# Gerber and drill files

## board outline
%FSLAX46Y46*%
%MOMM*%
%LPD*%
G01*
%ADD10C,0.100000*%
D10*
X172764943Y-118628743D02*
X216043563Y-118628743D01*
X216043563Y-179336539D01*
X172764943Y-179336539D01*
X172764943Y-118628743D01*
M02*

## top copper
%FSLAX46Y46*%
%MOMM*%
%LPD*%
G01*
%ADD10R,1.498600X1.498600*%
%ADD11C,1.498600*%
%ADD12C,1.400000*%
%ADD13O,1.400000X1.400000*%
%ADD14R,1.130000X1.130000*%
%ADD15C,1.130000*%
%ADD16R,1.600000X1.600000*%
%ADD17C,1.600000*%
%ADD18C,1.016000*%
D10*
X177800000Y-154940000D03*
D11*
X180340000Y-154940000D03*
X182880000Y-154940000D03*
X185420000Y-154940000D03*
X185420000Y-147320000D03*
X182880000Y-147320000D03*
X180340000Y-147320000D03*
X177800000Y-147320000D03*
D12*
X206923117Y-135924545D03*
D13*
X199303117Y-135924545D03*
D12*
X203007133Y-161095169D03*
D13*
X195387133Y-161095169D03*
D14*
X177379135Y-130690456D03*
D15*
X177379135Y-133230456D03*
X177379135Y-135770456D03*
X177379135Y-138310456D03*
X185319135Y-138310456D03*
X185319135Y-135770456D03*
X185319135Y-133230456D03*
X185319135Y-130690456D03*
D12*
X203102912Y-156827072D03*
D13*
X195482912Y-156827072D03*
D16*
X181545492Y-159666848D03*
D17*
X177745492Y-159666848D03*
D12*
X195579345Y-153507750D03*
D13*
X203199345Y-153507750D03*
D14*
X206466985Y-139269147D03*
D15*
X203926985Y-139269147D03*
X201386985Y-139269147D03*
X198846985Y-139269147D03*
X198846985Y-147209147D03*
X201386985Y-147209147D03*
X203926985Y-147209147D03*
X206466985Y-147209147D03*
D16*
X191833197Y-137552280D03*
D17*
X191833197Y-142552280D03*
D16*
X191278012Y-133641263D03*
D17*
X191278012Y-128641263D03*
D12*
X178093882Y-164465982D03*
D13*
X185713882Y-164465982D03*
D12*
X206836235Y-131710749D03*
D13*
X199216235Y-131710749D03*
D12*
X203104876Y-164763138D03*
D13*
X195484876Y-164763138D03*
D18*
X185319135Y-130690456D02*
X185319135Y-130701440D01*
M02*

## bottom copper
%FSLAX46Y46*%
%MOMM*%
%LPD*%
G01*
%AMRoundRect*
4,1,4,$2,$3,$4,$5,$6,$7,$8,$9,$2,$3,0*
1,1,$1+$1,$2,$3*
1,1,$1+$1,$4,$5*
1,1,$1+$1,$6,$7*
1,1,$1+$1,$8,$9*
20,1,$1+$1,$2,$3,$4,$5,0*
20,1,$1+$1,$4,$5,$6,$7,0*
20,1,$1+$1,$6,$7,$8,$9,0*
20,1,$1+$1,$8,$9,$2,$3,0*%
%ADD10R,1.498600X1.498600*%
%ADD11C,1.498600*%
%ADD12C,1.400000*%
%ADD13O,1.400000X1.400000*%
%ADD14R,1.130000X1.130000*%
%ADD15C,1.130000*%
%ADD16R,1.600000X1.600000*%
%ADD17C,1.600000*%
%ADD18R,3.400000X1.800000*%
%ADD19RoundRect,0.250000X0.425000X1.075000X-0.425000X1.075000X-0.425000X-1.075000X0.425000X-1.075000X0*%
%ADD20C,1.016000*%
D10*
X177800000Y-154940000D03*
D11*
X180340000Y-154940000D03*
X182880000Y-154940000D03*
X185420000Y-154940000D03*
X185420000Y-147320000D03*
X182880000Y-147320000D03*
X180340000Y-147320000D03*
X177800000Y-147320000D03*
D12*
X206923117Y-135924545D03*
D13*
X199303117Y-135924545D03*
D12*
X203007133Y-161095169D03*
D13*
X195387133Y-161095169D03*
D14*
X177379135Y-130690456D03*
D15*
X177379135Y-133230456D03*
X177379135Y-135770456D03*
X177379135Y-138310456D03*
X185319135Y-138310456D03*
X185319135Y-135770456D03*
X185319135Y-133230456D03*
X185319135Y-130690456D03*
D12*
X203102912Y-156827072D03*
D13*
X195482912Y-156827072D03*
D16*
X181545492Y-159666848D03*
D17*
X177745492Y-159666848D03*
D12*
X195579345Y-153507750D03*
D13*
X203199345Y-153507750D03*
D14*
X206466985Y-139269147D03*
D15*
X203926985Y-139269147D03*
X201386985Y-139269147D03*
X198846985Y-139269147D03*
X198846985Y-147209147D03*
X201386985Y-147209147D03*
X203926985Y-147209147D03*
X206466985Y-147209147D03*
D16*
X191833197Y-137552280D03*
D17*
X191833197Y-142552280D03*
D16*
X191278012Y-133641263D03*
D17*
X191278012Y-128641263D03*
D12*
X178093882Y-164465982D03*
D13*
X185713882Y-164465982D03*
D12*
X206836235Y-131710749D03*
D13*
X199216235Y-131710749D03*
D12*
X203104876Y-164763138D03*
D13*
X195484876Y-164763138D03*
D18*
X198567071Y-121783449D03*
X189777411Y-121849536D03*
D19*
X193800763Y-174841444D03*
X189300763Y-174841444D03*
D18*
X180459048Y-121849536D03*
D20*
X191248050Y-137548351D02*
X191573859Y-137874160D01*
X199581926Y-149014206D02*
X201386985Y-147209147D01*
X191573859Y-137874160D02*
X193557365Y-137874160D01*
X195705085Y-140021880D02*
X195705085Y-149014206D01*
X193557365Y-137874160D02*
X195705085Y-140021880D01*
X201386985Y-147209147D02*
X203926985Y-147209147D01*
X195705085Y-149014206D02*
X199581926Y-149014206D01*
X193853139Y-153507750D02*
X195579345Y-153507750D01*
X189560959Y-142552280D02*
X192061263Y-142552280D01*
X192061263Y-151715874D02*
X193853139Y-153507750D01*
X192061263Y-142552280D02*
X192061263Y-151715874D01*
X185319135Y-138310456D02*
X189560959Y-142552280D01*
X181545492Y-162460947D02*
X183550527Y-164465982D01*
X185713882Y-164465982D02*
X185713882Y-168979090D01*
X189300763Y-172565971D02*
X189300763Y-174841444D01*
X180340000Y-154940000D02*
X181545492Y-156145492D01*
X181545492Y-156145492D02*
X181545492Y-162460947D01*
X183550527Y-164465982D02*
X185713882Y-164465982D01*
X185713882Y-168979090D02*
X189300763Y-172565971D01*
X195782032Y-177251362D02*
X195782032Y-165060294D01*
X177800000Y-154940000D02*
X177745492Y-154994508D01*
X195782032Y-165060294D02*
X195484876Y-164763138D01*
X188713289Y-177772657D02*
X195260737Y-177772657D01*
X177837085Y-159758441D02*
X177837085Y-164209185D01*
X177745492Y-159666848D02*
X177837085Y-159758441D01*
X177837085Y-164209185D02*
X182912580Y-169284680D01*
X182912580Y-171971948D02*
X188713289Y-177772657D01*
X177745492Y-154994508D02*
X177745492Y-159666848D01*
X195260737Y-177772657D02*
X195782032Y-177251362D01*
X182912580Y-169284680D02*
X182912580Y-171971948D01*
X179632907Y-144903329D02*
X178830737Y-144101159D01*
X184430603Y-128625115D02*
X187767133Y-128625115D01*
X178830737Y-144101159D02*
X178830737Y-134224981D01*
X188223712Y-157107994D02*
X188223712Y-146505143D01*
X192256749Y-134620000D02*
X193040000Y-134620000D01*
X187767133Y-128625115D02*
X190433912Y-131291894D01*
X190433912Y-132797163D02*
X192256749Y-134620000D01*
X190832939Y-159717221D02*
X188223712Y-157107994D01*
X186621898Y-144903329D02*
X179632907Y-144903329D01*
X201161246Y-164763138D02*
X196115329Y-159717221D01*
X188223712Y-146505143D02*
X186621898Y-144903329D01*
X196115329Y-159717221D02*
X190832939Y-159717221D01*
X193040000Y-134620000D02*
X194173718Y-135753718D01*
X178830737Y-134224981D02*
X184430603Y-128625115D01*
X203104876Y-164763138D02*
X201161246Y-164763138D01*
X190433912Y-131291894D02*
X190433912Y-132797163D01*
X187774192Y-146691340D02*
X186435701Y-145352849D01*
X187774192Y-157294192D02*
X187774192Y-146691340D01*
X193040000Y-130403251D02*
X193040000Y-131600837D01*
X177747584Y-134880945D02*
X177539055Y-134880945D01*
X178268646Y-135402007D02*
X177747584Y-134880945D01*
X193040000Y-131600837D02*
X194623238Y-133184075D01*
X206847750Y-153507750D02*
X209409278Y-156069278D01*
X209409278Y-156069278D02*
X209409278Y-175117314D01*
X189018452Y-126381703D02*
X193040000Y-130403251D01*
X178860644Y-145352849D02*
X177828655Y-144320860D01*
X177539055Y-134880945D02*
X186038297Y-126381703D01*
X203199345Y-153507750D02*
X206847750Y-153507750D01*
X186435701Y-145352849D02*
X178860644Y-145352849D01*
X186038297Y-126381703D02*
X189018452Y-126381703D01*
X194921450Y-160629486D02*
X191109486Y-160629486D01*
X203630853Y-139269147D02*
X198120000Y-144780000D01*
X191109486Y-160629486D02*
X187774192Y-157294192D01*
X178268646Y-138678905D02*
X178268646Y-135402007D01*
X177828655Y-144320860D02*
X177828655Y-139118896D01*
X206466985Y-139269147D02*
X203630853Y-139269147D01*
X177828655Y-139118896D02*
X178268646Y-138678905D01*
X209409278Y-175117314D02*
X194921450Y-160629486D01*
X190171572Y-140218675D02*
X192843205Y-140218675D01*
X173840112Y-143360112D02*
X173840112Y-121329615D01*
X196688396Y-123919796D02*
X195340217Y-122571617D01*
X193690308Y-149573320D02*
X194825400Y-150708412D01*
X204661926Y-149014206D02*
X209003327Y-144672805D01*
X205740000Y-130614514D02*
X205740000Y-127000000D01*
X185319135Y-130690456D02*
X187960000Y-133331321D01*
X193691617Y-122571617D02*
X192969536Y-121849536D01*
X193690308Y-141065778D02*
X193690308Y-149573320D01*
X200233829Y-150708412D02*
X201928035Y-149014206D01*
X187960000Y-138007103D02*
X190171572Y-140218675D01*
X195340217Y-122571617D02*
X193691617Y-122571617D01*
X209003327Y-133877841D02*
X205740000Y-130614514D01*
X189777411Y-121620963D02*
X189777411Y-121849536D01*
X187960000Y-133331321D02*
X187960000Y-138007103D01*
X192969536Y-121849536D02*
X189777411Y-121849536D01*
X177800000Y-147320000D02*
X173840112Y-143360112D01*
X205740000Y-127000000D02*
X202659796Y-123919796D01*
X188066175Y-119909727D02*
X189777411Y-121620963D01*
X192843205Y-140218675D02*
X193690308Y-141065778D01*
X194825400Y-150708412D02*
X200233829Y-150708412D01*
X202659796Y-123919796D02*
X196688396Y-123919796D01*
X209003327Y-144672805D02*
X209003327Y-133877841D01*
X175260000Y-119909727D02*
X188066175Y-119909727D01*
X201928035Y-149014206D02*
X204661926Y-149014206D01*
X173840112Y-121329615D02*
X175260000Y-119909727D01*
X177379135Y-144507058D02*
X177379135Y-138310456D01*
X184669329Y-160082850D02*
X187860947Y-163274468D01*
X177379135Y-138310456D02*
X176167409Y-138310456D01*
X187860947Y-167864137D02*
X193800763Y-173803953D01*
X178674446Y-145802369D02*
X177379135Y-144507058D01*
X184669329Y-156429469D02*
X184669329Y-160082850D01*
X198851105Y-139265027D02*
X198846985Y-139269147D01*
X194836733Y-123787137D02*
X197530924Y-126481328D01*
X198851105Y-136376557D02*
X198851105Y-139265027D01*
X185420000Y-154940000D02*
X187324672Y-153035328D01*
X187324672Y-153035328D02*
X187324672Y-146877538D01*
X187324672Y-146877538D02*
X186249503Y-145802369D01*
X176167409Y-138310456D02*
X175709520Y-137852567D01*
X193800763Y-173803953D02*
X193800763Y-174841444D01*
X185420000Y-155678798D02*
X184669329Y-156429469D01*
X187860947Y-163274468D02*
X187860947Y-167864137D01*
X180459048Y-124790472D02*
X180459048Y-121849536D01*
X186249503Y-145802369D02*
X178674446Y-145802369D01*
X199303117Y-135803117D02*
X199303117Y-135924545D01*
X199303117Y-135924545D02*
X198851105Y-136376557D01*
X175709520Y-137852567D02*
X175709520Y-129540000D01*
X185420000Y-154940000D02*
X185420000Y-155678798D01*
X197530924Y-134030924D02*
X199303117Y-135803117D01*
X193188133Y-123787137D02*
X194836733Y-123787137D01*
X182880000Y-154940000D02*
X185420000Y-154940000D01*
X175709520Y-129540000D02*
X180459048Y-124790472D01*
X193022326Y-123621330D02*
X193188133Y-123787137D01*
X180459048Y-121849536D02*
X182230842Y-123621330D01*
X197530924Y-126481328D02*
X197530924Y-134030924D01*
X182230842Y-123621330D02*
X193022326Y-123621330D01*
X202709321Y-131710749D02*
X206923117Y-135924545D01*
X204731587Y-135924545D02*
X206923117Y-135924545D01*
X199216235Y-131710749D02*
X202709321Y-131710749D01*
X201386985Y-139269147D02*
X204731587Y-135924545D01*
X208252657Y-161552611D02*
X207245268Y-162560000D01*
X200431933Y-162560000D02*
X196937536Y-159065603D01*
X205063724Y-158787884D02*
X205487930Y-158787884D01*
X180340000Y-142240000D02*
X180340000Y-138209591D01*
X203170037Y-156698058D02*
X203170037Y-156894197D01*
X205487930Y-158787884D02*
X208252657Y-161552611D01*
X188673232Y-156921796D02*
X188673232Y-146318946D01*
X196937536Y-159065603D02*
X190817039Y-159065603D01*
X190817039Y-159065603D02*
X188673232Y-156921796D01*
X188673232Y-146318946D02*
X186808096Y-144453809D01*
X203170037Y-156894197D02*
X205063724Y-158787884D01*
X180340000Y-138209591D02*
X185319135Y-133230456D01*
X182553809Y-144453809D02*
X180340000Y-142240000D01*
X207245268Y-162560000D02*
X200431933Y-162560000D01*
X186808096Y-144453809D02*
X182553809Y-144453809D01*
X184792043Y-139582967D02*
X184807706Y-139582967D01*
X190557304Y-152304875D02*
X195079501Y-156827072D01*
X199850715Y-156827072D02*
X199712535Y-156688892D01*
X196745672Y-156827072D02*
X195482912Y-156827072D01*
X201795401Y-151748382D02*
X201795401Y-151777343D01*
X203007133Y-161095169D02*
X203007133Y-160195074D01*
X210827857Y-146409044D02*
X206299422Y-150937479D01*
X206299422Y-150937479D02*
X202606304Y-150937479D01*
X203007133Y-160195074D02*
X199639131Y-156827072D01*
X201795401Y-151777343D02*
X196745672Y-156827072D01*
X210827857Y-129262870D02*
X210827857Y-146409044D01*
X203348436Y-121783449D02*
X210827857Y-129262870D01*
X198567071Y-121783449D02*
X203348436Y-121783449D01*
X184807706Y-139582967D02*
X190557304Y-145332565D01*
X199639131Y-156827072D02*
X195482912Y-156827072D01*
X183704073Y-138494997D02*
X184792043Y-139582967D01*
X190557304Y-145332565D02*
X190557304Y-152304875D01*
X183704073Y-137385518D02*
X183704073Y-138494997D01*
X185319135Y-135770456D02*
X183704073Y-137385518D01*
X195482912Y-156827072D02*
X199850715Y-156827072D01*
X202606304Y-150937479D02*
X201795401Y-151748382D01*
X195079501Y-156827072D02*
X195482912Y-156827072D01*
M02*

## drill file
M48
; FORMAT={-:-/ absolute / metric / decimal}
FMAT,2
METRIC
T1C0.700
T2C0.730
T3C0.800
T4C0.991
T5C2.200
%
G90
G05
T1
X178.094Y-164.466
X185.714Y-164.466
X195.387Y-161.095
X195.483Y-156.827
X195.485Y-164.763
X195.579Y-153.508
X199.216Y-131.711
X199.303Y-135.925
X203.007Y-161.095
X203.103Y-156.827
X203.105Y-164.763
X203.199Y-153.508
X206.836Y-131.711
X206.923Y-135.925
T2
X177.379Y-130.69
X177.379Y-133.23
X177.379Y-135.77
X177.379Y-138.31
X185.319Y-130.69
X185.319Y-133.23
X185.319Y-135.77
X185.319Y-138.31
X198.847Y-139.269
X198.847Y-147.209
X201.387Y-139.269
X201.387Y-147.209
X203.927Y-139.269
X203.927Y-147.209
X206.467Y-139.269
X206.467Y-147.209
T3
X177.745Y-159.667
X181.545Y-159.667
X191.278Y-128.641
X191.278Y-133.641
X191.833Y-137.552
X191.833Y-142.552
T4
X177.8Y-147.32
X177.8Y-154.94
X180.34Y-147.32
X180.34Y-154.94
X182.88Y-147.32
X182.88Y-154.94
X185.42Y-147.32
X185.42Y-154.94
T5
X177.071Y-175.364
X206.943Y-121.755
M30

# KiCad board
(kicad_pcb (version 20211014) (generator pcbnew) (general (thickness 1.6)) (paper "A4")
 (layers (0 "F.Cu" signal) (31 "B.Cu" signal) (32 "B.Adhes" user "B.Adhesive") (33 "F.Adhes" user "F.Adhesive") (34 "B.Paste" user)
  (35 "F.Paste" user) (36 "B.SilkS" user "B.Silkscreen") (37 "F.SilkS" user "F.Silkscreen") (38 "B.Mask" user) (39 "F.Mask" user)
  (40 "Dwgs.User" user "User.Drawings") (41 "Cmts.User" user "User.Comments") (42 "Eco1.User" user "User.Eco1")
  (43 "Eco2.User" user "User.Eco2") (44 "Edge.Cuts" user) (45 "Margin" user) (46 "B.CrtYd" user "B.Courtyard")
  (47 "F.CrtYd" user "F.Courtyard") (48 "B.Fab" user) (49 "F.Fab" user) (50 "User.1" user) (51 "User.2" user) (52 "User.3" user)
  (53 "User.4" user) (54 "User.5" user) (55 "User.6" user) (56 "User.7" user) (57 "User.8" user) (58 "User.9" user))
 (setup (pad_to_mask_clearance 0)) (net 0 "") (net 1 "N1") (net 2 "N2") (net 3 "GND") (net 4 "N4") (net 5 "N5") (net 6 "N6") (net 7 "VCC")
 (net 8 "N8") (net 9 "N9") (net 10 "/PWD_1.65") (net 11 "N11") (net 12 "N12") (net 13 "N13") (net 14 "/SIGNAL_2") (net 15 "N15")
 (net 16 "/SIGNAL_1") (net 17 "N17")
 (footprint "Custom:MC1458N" (layer "F.Cu") (at 177.8 154.94 90)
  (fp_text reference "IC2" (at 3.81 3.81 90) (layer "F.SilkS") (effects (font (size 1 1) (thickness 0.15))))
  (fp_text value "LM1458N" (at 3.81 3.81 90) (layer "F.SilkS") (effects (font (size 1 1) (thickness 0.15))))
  (pad "1" thru_hole rect locked (at 0 0 90) (size 1.4986 1.4986) (drill 0.9906) (layers *.Cu *.Mask) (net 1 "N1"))
  (pad "2" thru_hole circle locked (at 0 2.54 90) (size 1.4986 1.4986) (drill 0.9906) (layers *.Cu *.Mask) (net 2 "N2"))
  (pad "3" thru_hole circle locked (at 0 5.08 90) (size 1.4986 1.4986) (drill 0.9906) (layers *.Cu *.Mask) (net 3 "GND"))
  (pad "4" thru_hole circle locked (at 0 7.62 90) (size 1.4986 1.4986) (drill 0.9906) (layers *.Cu *.Mask) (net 3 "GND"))
  (pad "5" thru_hole circle locked (at 7.62 7.62 90) (size 1.4986 1.4986) (drill 0.9906) (layers *.Cu *.Mask) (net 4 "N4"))
  (pad "6" thru_hole circle locked (at 7.62 5.08 90) (size 1.4986 1.4986) (drill 0.9906) (layers *.Cu *.Mask) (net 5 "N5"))
  (pad "7" thru_hole circle locked (at 7.62 2.54 90) (size 1.4986 1.4986) (drill 0.9906) (layers *.Cu *.Mask) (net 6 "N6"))
  (pad "8" thru_hole circle locked (at 7.62 0 90) (size 1.4986 1.4986) (drill 0.9906) (layers *.Cu *.Mask) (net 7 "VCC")))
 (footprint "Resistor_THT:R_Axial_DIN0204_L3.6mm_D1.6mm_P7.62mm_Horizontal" (layer "F.Cu") (at 206.923117 135.924545 180)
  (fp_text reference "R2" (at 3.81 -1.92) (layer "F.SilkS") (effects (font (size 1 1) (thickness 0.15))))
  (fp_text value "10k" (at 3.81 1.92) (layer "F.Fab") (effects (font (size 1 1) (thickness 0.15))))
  (pad "1" thru_hole circle (at 0 0 180) (size 1.4 1.4) (drill 0.7) (layers *.Cu *.Mask) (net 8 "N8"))
  (pad "2" thru_hole oval (at 7.62 0 180) (size 1.4 1.4) (drill 0.7) (layers *.Cu *.Mask) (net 3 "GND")))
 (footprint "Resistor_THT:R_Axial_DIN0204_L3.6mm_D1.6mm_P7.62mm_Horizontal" (layer "F.Cu") (at 203.007133 161.095169 180)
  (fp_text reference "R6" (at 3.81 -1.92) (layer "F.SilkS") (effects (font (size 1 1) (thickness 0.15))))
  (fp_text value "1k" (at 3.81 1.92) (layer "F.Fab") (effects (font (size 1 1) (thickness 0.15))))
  (pad "1" thru_hole circle (at 0 0 180) (size 1.4 1.4) (drill 0.7) (layers *.Cu *.Mask) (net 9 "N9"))
  (pad "2" thru_hole oval (at 7.62 0 180) (size 1.4 1.4) (drill 0.7) (layers *.Cu *.Mask) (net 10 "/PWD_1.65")))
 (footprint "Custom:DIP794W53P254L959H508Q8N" (layer "F.Cu") (at 181.349135 134.500456)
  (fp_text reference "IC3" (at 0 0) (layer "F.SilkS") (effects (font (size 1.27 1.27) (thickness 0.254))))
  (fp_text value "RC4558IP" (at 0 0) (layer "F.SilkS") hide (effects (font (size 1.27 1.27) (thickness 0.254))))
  (pad "1" thru_hole rect locked (at -3.97 -3.81) (size 1.13 1.13) (drill 0.73) (layers *.Cu *.Mask) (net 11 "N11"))
  (pad "2" thru_hole circle locked (at -3.97 -1.27) (size 1.13 1.13) (drill 0.73) (layers *.Cu *.Mask) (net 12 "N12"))
  (pad "3" thru_hole circle locked (at -3.97 1.27) (size 1.13 1.13) (drill 0.73) (layers *.Cu *.Mask) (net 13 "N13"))
  (pad "4" thru_hole circle locked (at -3.97 3.81) (size 1.13 1.13) (drill 0.73) (layers *.Cu *.Mask) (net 3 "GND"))
  (pad "5" thru_hole circle locked (at 3.97 3.81) (size 1.13 1.13) (drill 0.73) (layers *.Cu *.Mask) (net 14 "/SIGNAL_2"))
  (pad "6" thru_hole circle locked (at 3.97 1.27) (size 1.13 1.13) (drill 0.73) (layers *.Cu *.Mask) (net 9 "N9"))
  (pad "7" thru_hole circle locked (at 3.97 -1.27) (size 1.13 1.13) (drill 0.73) (layers *.Cu *.Mask) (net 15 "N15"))
  (pad "8" thru_hole circle locked (at 3.97 -3.81) (size 1.13 1.13) (drill 0.73) (layers *.Cu *.Mask) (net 7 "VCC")))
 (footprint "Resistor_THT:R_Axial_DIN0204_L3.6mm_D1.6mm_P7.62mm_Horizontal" (layer "F.Cu") (at 203.102912 156.827072 180)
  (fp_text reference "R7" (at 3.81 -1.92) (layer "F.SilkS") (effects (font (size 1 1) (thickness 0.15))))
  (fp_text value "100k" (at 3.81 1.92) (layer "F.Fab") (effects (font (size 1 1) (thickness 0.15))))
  (pad "1" thru_hole circle (at 0 0 180) (size 1.4 1.4) (drill 0.7) (layers *.Cu *.Mask) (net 15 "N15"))
  (pad "2" thru_hole oval (at 7.62 0 180) (size 1.4 1.4) (drill 0.7) (layers *.Cu *.Mask) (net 9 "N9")))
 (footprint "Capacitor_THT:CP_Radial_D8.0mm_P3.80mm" (layer "F.Cu") (at 181.545492 159.666848 180)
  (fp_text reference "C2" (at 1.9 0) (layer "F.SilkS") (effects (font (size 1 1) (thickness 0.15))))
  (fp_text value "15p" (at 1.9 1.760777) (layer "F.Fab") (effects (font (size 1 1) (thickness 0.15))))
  (pad "1" thru_hole rect (at 0 0 180) (size 1.6 1.6) (drill 0.8) (layers *.Cu *.Mask) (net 2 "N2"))
  (pad "2" thru_hole circle (at 3.8 0 180) (size 1.6 1.6) (drill 0.8) (layers *.Cu *.Mask) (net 1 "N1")))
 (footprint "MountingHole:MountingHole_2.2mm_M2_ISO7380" (layer "F.Cu") (at 206.942704 121.75478)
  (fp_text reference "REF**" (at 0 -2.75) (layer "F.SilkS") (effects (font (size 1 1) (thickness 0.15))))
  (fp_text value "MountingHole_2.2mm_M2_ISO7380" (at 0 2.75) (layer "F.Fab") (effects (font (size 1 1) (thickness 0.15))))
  (pad "" np_thru_hole circle (at 0 0) (size 2.2 2.2) (drill 2.2) (layers *.Cu *.Mask)))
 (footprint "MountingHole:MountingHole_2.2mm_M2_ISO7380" (layer "F.Cu") (at 177.071075 175.363506)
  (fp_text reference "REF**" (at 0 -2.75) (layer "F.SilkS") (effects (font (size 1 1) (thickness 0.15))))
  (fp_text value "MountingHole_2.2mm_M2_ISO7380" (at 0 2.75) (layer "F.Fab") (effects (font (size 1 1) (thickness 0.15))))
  (pad "" np_thru_hole circle (at 0 0) (size 2.2 2.2) (drill 2.2) (layers *.Cu *.Mask)))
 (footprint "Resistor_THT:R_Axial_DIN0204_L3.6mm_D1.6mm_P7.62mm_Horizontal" (layer "F.Cu") (at 195.579345 153.50775)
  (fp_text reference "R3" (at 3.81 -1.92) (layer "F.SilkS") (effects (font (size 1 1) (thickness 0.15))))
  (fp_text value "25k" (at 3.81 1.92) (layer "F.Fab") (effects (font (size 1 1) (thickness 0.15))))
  (pad "1" thru_hole circle (at 0 0) (size 1.4 1.4) (drill 0.7) (layers *.Cu *.Mask) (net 14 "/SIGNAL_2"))
  (pad "2" thru_hole oval (at 7.62 0) (size 1.4 1.4) (drill 0.7) (layers *.Cu *.Mask) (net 10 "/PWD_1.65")))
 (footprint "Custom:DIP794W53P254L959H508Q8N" (layer "F.Cu") (at 202.656985 143.239147 -90)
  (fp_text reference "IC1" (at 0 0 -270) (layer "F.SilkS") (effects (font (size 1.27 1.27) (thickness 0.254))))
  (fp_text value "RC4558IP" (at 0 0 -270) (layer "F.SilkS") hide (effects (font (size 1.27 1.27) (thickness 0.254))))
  (pad "1" thru_hole rect locked (at -3.97 -3.81 270) (size 1.13 1.13) (drill 0.73) (layers *.Cu *.Mask) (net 10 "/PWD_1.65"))
  (pad "2" thru_hole circle locked (at -3.97 -1.27 270) (size 1.13 1.13) (drill 0.73) (layers *.Cu *.Mask) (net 10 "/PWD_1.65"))
  (pad "3" thru_hole circle locked (at -3.97 1.27 270) (size 1.13 1.13) (drill 0.73) (layers *.Cu *.Mask) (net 8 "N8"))
  (pad "4" thru_hole circle locked (at -3.97 3.81 270) (size 1.13 1.13) (drill 0.73) (layers *.Cu *.Mask) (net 3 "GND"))
  (pad "5" thru_hole circle locked (at 3.97 3.81 270) (size 1.13 1.13) (drill 0.73) (layers *.Cu *.Mask) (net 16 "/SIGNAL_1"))
  (pad "6" thru_hole circle locked (at 3.97 1.27 270) (size 1.13 1.13) (drill 0.73) (layers *.Cu *.Mask) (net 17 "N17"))
  (pad "7" thru_hole circle locked (at 3.97 -1.27 270) (size 1.13 1.13) (drill 0.73) (layers *.Cu *.Mask) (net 17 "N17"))
  (pad "8" thru_hole circle locked (at 3.97 -3.81 270) (size 1.13 1.13) (drill 0.73) (layers *.Cu *.Mask) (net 7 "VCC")))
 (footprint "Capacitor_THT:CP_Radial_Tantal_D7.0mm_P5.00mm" (layer "F.Cu") (at 191.833197 137.55228 -90)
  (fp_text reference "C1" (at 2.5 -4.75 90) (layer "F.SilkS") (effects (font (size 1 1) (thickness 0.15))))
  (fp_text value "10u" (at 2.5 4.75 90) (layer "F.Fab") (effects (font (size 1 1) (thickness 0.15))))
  (pad "1" thru_hole rect (at 0 0 270) (size 1.6 1.6) (drill 0.8) (layers *.Cu *.Mask) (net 17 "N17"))
  (pad "2" thru_hole circle (at 5 0 270) (size 1.6 1.6) (drill 0.8) (layers *.Cu *.Mask) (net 14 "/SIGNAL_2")))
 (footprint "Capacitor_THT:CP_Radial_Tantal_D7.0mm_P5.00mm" (layer "F.Cu") (at 191.278012 133.641263 90)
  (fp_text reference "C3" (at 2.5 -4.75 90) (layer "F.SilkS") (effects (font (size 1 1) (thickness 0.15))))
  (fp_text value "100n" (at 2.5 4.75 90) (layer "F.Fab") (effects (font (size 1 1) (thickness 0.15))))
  (pad "1" thru_hole rect (at 0 0 90) (size 1.6 1.6) (drill 0.8) (layers *.Cu *.Mask) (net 16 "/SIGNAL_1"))
  (pad "2" thru_hole circle (at 5 0 90) (size 1.6 1.6) (drill 0.8) (layers *.Cu *.Mask) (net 10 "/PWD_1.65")))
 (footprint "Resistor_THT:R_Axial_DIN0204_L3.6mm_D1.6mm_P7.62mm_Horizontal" (layer "F.Cu") (at 178.093882 164.465982)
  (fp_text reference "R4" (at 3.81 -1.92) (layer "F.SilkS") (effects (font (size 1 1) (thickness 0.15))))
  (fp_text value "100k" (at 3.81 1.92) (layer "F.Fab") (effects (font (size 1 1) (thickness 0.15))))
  (pad "1" thru_hole circle (at 0 0) (size 1.4 1.4) (drill 0.7) (layers *.Cu *.Mask) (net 1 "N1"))
  (pad "2" thru_hole oval (at 7.62 0) (size 1.4 1.4) (drill 0.7) (layers *.Cu *.Mask) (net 2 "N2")))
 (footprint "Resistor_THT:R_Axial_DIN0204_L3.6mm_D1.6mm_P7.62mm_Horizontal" (layer "F.Cu") (at 206.836235 131.710749 180)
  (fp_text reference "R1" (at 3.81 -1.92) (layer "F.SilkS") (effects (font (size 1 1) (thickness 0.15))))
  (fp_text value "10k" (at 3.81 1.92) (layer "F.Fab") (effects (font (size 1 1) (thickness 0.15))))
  (pad "1" thru_hole circle (at 0 0 180) (size 1.4 1.4) (drill 0.7) (layers *.Cu *.Mask) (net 7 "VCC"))
  (pad "2" thru_hole oval (at 7.62 0 180) (size 1.4 1.4) (drill 0.7) (layers *.Cu *.Mask) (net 8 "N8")))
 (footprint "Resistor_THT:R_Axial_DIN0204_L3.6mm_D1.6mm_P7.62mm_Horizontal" (layer "F.Cu") (at 203.104876 164.763138 180)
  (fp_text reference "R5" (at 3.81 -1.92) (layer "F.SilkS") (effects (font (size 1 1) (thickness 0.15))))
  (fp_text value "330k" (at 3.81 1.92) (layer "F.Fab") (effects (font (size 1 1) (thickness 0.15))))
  (pad "1" thru_hole circle (at 0 0 180) (size 1.4 1.4) (drill 0.7) (layers *.Cu *.Mask) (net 16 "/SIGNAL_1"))
  (pad "2" thru_hole oval (at 7.62 0 180) (size 1.4 1.4) (drill 0.7) (layers *.Cu *.Mask) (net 1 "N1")))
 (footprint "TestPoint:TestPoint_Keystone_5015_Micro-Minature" (layer "B.Cu") (at 198.567071 121.783449)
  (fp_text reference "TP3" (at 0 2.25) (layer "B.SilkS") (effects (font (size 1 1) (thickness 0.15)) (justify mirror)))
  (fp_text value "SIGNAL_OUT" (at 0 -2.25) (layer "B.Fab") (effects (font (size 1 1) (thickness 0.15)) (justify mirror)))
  (pad "1" smd rect (at 0 0) (size 3.4 1.8) (layers "B.Cu" "B.Paste" "B.Mask") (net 9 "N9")))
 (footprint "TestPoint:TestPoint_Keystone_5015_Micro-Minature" (layer "B.Cu") (at 189.777411 121.849536)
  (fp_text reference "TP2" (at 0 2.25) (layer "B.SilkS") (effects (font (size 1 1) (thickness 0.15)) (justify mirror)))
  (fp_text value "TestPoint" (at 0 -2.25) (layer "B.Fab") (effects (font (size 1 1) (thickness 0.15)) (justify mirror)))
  (pad "1" smd rect (at 0 0) (size 3.4 1.8) (layers "B.Cu" "B.Paste" "B.Mask") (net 7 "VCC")))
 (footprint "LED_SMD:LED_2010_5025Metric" (layer "B.Cu") (at 191.550763 174.841444 180)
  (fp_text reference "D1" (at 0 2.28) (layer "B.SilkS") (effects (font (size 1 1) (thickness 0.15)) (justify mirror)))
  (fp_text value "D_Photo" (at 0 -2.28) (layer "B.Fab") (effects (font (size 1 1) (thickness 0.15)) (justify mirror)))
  (pad "1" smd roundrect (at -2.25 0 180) (size 1.35 2.65) (layers "B.Cu" "B.Paste" "B.Mask") (roundrect_rratio 0.185185) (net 3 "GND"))
  (pad "2" smd roundrect (at 2.25 0 180) (size 1.35 2.65) (layers "B.Cu" "B.Paste" "B.Mask") (roundrect_rratio 0.185185) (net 2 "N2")))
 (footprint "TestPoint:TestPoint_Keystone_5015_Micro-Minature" (layer "B.Cu") (at 180.459048 121.849536)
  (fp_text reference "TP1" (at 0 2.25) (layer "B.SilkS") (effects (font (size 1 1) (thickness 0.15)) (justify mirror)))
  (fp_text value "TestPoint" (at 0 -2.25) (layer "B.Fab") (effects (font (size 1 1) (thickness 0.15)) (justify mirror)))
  (pad "1" smd rect (at 0 0) (size 3.4 1.8) (layers "B.Cu" "B.Paste" "B.Mask") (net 3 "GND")))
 (gr_rect (start 216.043563 179.336539) (end 172.764943 118.628743) (layer "Edge.Cuts") (width 0.1) (fill none))
 (segment (start 191.24805 137.548351) (end 191.573859 137.87416) (width 1.016) (layer "B.Cu") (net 17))
 (segment (start 199.581926 149.014206) (end 201.386985 147.209147) (width 1.016) (layer "B.Cu") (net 17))
 (segment (start 191.573859 137.87416) (end 193.557365 137.87416) (width 1.016) (layer "B.Cu") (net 17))
 (segment (start 195.705085 140.02188) (end 195.705085 149.014206) (width 1.016) (layer "B.Cu") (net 17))
 (segment (start 193.557365 137.87416) (end 195.705085 140.02188) (width 1.016) (layer "B.Cu") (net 17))
 (segment (start 201.386985 147.209147) (end 203.926985 147.209147) (width 1.016) (layer "B.Cu") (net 17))
 (segment (start 195.705085 149.014206) (end 199.581926 149.014206) (width 1.016) (layer "B.Cu") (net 17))
 (segment (start 193.853139 153.50775) (end 195.579345 153.50775) (width 1.016) (layer "B.Cu") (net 14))
 (segment (start 189.560959 142.55228) (end 192.061263 142.55228) (width 1.016) (layer "B.Cu") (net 14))
 (segment (start 192.061263 151.715874) (end 193.853139 153.50775) (width 1.016) (layer "B.Cu") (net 14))
 (segment (start 192.061263 142.55228) (end 192.061263 151.715874) (width 1.016) (layer "B.Cu") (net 14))
 (segment (start 185.319135 138.310456) (end 189.560959 142.55228) (width 1.016) (layer "B.Cu") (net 14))
 (segment (start 181.545492 162.460947) (end 183.550527 164.465982) (width 1.016) (layer "B.Cu") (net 2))
 (segment (start 185.713882 164.465982) (end 185.713882 168.97909) (width 1.016) (layer "B.Cu") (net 2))
 (segment (start 189.300763 172.565971) (end 189.300763 174.841444) (width 1.016) (layer "B.Cu") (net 2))
 (segment (start 180.34 154.94) (end 181.545492 156.145492) (width 1.016) (layer "B.Cu") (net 2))
 (segment (start 181.545492 156.145492) (end 181.545492 162.460947) (width 1.016) (layer "B.Cu") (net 2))
 (segment (start 183.550527 164.465982) (end 185.713882 164.465982) (width 1.016) (layer "B.Cu") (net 2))
 (segment (start 185.713882 168.97909) (end 189.300763 172.565971) (width 1.016) (layer "B.Cu") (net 2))
 (segment (start 195.782032 177.251362) (end 195.782032 165.060294) (width 1.016) (layer "B.Cu") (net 1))
 (segment (start 177.8 154.94) (end 177.745492 154.994508) (width 1.016) (layer "B.Cu") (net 1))
 (segment (start 195.782032 165.060294) (end 195.484876 164.763138) (width 1.016) (layer "B.Cu") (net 1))
 (segment (start 188.713289 177.772657) (end 195.260737 177.772657) (width 1.016) (layer "B.Cu") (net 1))
 (segment (start 177.837085 159.758441) (end 177.837085 164.209185) (width 1.016) (layer "B.Cu") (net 1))
 (segment (start 177.745492 159.666848) (end 177.837085 159.758441) (width 1.016) (layer "B.Cu") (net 1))
 (segment (start 177.837085 164.209185) (end 182.91258 169.28468) (width 1.016) (layer "B.Cu") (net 1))
 (segment (start 182.91258 171.971948) (end 188.713289 177.772657) (width 1.016) (layer "B.Cu") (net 1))
 (segment (start 177.745492 154.994508) (end 177.745492 159.666848) (width 1.016) (layer "B.Cu") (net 1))
 (segment (start 195.260737 177.772657) (end 195.782032 177.251362) (width 1.016) (layer "B.Cu") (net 1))
 (segment (start 182.91258 169.28468) (end 182.91258 171.971948) (width 1.016) (layer "B.Cu") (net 1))
 (segment (start 179.632907 144.903329) (end 178.830737 144.101159) (width 1.016) (layer "B.Cu") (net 16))
 (segment (start 184.430603 128.625115) (end 187.767133 128.625115) (width 1.016) (layer "B.Cu") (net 16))
 (segment (start 178.830737 144.101159) (end 178.830737 134.224981) (width 1.016) (layer "B.Cu") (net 16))
 (segment (start 188.223712 157.107994) (end 188.223712 146.505143) (width 1.016) (layer "B.Cu") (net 16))
 (segment (start 192.256749 134.62) (end 193.04 134.62) (width 1.016) (layer "B.Cu") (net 16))
 (segment (start 187.767133 128.625115) (end 190.433912 131.291894) (width 1.016) (layer "B.Cu") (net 16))
 (segment (start 190.433912 132.797163) (end 192.256749 134.62) (width 1.016) (layer "B.Cu") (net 16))
 (segment (start 190.832939 159.717221) (end 188.223712 157.107994) (width 1.016) (layer "B.Cu") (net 16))
 (segment (start 186.621898 144.903329) (end 179.632907 144.903329) (width 1.016) (layer "B.Cu") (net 16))
 (segment (start 201.161246 164.763138) (end 196.115329 159.717221) (width 1.016) (layer "B.Cu") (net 16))
 (segment (start 188.223712 146.505143) (end 186.621898 144.903329) (width 1.016) (layer "B.Cu") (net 16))
 (segment (start 196.115329 159.717221) (end 190.832939 159.717221) (width 1.016) (layer "B.Cu") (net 16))
 (segment (start 193.04 134.62) (end 194.173718 135.753718) (width 1.016) (layer "B.Cu") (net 16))
 (segment (start 178.830737 134.224981) (end 184.430603 128.625115) (width 1.016) (layer "B.Cu") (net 16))
 (segment (start 203.104876 164.763138) (end 201.161246 164.763138) (width 1.016) (layer "B.Cu") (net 16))
 (segment (start 190.433912 131.291894) (end 190.433912 132.797163) (width 1.016) (layer "B.Cu") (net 16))
 (segment (start 187.774192 146.69134) (end 186.435701 145.352849) (width 1.016) (layer "B.Cu") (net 10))
 (segment (start 187.774192 157.294192) (end 187.774192 146.69134) (width 1.016) (layer "B.Cu") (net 10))
 (segment (start 193.04 130.403251) (end 193.04 131.600837) (width 1.016) (layer "B.Cu") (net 10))
 (segment (start 177.747584 134.880945) (end 177.539055 134.880945) (width 1.016) (layer "B.Cu") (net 10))
 (segment (start 178.268646 135.402007) (end 177.747584 134.880945) (width 1.016) (layer "B.Cu") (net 10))
 (segment (start 193.04 131.600837) (end 194.623238 133.184075) (width 1.016) (layer "B.Cu") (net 10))
 (segment (start 206.84775 153.50775) (end 209.409278 156.069278) (width 1.016) (layer "B.Cu") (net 10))
 (segment (start 209.409278 156.069278) (end 209.409278 175.117314) (width 1.016) (layer "B.Cu") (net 10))
 (segment (start 189.018452 126.381703) (end 193.04 130.403251) (width 1.016) (layer "B.Cu") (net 10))
 (segment (start 178.860644 145.352849) (end 177.828655 144.32086) (width 1.016) (layer "B.Cu") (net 10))
 (segment (start 177.539055 134.880945) (end 186.038297 126.381703) (width 1.016) (layer "B.Cu") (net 10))
 (segment (start 203.199345 153.50775) (end 206.84775 153.50775) (width 1.016) (layer "B.Cu") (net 10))
 (segment (start 186.435701 145.352849) (end 178.860644 145.352849) (width 1.016) (layer "B.Cu") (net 10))
 (segment (start 186.038297 126.381703) (end 189.018452 126.381703) (width 1.016) (layer "B.Cu") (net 10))
 (segment (start 194.92145 160.629486) (end 191.109486 160.629486) (width 1.016) (layer "B.Cu") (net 10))
 (segment (start 203.630853 139.269147) (end 198.12 144.78) (width 1.016) (layer "B.Cu") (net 10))
 (segment (start 191.109486 160.629486) (end 187.774192 157.294192) (width 1.016) (layer "B.Cu") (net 10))
 (segment (start 178.268646 138.678905) (end 178.268646 135.402007) (width 1.016) (layer "B.Cu") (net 10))
 (segment (start 177.828655 144.32086) (end 177.828655 139.118896) (width 1.016) (layer "B.Cu") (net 10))
 (segment (start 206.466985 139.269147) (end 203.630853 139.269147) (width 1.016) (layer "B.Cu") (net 10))
 (segment (start 177.828655 139.118896) (end 178.268646 138.678905) (width 1.016) (layer "B.Cu") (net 10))
 (segment (start 209.409278 175.117314) (end 194.92145 160.629486) (width 1.016) (layer "B.Cu") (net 10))
 (segment (start 185.319135 130.690456) (end 185.319135 130.70144) (width 1.016) (layer "F.Cu") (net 7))
 (segment (start 190.171572 140.218675) (end 192.843205 140.218675) (width 1.016) (layer "B.Cu") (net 7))
 (segment (start 173.840112 143.360112) (end 173.840112 121.329615) (width 1.016) (layer "B.Cu") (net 7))
 (segment (start 196.688396 123.919796) (end 195.340217 122.571617) (width 1.016) (layer "B.Cu") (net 7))
 (segment (start 193.690308 149.57332) (end 194.8254 150.708412) (width 1.016) (layer "B.Cu") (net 7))
 (segment (start 204.661926 149.014206) (end 209.003327 144.672805) (width 1.016) (layer "B.Cu") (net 7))
 (segment (start 205.74 130.614514) (end 205.74 127) (width 1.016) (layer "B.Cu") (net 7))
 (segment (start 185.319135 130.690456) (end 187.96 133.331321) (width 1.016) (layer "B.Cu") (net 7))
 (segment (start 193.691617 122.571617) (end 192.969536 121.849536) (width 1.016) (layer "B.Cu") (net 7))
 (segment (start 193.690308 141.065778) (end 193.690308 149.57332) (width 1.016) (layer "B.Cu") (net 7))
 (segment (start 200.233829 150.708412) (end 201.928035 149.014206) (width 1.016) (layer "B.Cu") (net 7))
 (segment (start 187.96 138.007103) (end 190.171572 140.218675) (width 1.016) (layer "B.Cu") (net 7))
 (segment (start 195.340217 122.571617) (end 193.691617 122.571617) (width 1.016) (layer "B.Cu") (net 7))
 (segment (start 209.003327 133.877841) (end 205.74 130.614514) (width 1.016) (layer "B.Cu") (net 7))
 (segment (start 189.777411 121.620963) (end 189.777411 121.849536) (width 1.016) (layer "B.Cu") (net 7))
 (segment (start 187.96 133.331321) (end 187.96 138.007103) (width 1.016) (layer "B.Cu") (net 7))
 (segment (start 192.969536 121.849536) (end 189.777411 121.849536) (width 1.016) (layer "B.Cu") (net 7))
 (segment (start 177.8 147.32) (end 173.840112 143.360112) (width 1.016) (layer "B.Cu") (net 7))
 (segment (start 205.74 127) (end 202.659796 123.919796) (width 1.016) (layer "B.Cu") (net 7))
 (segment (start 188.066175 119.909727) (end 189.777411 121.620963) (width 1.016) (layer "B.Cu") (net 7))
 (segment (start 192.843205 140.218675) (end 193.690308 141.065778) (width 1.016) (layer "B.Cu") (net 7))
 (segment (start 194.8254 150.708412) (end 200.233829 150.708412) (width 1.016) (layer "B.Cu") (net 7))
 (segment (start 202.659796 123.919796) (end 196.688396 123.919796) (width 1.016) (layer "B.Cu") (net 7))
 (segment (start 209.003327 144.672805) (end 209.003327 133.877841) (width 1.016) (layer "B.Cu") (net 7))
 (segment (start 175.26 119.909727) (end 188.066175 119.909727) (width 1.016) (layer "B.Cu") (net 7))
 (segment (start 201.928035 149.014206) (end 204.661926 149.014206) (width 1.016) (layer "B.Cu") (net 7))
 (segment (start 173.840112 121.329615) (end 175.26 119.909727) (width 1.016) (layer "B.Cu") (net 7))
 (segment (start 177.379135 144.507058) (end 177.379135 138.310456) (width 1.016) (layer "B.Cu") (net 3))
 (segment (start 184.669329 160.08285) (end 187.860947 163.274468) (width 1.016) (layer "B.Cu") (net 3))
 (segment (start 177.379135 138.310456) (end 176.167409 138.310456) (width 1.016) (layer "B.Cu") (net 3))
 (segment (start 187.860947 167.864137) (end 193.800763 173.803953) (width 1.016) (layer "B.Cu") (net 3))
 (segment (start 178.674446 145.802369) (end 177.379135 144.507058) (width 1.016) (layer "B.Cu") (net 3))
 (segment (start 184.669329 156.429469) (end 184.669329 160.08285) (width 1.016) (layer "B.Cu") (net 3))
 (segment (start 198.851105 139.265027) (end 198.846985 139.269147) (width 1.016) (layer "B.Cu") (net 3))
 (segment (start 194.836733 123.787137) (end 197.530924 126.481328) (width 1.016) (layer "B.Cu") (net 3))
 (segment (start 198.851105 136.376557) (end 198.851105 139.265027) (width 1.016) (layer "B.Cu") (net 3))
 (segment (start 185.42 154.94) (end 187.324672 153.035328) (width 1.016) (layer "B.Cu") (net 3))
 (segment (start 187.324672 153.035328) (end 187.324672 146.877538) (width 1.016) (layer "B.Cu") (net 3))
 (segment (start 187.324672 146.877538) (end 186.249503 145.802369) (width 1.016) (layer "B.Cu") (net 3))
 (segment (start 176.167409 138.310456) (end 175.70952 137.852567) (width 1.016) (layer "B.Cu") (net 3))
 (segment (start 193.800763 173.803953) (end 193.800763 174.841444) (width 1.016) (layer "B.Cu") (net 3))
 (segment (start 185.42 155.678798) (end 184.669329 156.429469) (width 1.016) (layer "B.Cu") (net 3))
 (segment (start 187.860947 163.274468) (end 187.860947 167.864137) (width 1.016) (layer "B.Cu") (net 3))
 (segment (start 180.459048 124.790472) (end 180.459048 121.849536) (width 1.016) (layer "B.Cu") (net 3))
 (segment (start 186.249503 145.802369) (end 178.674446 145.802369) (width 1.016) (layer "B.Cu") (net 3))
 (segment (start 199.303117 135.803117) (end 199.303117 135.924545) (width 1.016) (layer "B.Cu") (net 3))
 (segment (start 199.303117 135.924545) (end 198.851105 136.376557) (width 1.016) (layer "B.Cu") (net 3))
 (segment (start 175.70952 137.852567) (end 175.70952 129.54) (width 1.016) (layer "B.Cu") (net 3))
 (segment (start 185.42 154.94) (end 185.42 155.678798) (width 1.016) (layer "B.Cu") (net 3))
 (segment (start 197.530924 134.030924) (end 199.303117 135.803117) (width 1.016) (layer "B.Cu") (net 3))
 (segment (start 193.188133 123.787137) (end 194.836733 123.787137) (width 1.016) (layer "B.Cu") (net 3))
 (segment (start 182.88 154.94) (end 185.42 154.94) (width 1.016) (layer "B.Cu") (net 3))
 (segment (start 175.70952 129.54) (end 180.459048 124.790472) (width 1.016) (layer "B.Cu") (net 3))
 (segment (start 193.022326 123.62133) (end 193.188133 123.787137) (width 1.016) (layer "B.Cu") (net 3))
 (segment (start 180.459048 121.849536) (end 182.230842 123.62133) (width 1.016) (layer "B.Cu") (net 3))
 (segment (start 197.530924 126.481328) (end 197.530924 134.030924) (width 1.016) (layer "B.Cu") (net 3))
 (segment (start 182.230842 123.62133) (end 193.022326 123.62133) (width 1.016) (layer "B.Cu") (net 3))
 (segment (start 202.709321 131.710749) (end 206.923117 135.924545) (width 1.016) (layer "B.Cu") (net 8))
 (segment (start 204.731587 135.924545) (end 206.923117 135.924545) (width 1.016) (layer "B.Cu") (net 8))
 (segment (start 199.216235 131.710749) (end 202.709321 131.710749) (width 1.016) (layer "B.Cu") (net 8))
 (segment (start 201.386985 139.269147) (end 204.731587 135.924545) (width 1.016) (layer "B.Cu") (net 8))
 (segment (start 208.252657 161.552611) (end 207.245268 162.56) (width 1.016) (layer "B.Cu") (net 15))
 (segment (start 200.431933 162.56) (end 196.937536 159.065603) (width 1.016) (layer "B.Cu") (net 15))
 (segment (start 205.063724 158.787884) (end 205.48793 158.787884) (width 1.016) (layer "B.Cu") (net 15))
 (segment (start 180.34 142.24) (end 180.34 138.209591) (width 1.016) (layer "B.Cu") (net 15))
 (segment (start 203.170037 156.698058) (end 203.170037 156.894197) (width 1.016) (layer "B.Cu") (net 15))
 (segment (start 205.48793 158.787884) (end 208.252657 161.552611) (width 1.016) (layer "B.Cu") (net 15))
 (segment (start 188.673232 156.921796) (end 188.673232 146.318946) (width 1.016) (layer "B.Cu") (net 15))
 (segment (start 196.937536 159.065603) (end 190.817039 159.065603) (width 1.016) (layer "B.Cu") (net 15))
 (segment (start 190.817039 159.065603) (end 188.673232 156.921796) (width 1.016) (layer "B.Cu") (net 15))
 (segment (start 188.673232 146.318946) (end 186.808096 144.453809) (width 1.016) (layer "B.Cu") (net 15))
 (segment (start 203.170037 156.894197) (end 205.063724 158.787884) (width 1.016) (layer "B.Cu") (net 15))
 (segment (start 180.34 138.209591) (end 185.319135 133.230456) (width 1.016) (layer "B.Cu") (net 15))
 (segment (start 182.553809 144.453809) (end 180.34 142.24) (width 1.016) (layer "B.Cu") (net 15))
 (segment (start 207.245268 162.56) (end 200.431933 162.56) (width 1.016) (layer "B.Cu") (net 15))
 (segment (start 186.808096 144.453809) (end 182.553809 144.453809) (width 1.016) (layer "B.Cu") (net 15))
 (segment (start 184.792043 139.582967) (end 184.807706 139.582967) (width 1.016) (layer "B.Cu") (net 9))
 (segment (start 190.557304 152.304875) (end 195.079501 156.827072) (width 1.016) (layer "B.Cu") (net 9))
 (segment (start 199.850715 156.827072) (end 199.712535 156.688892) (width 1.016) (layer "B.Cu") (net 9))
 (segment (start 196.745672 156.827072) (end 195.482912 156.827072) (width 1.016) (layer "B.Cu") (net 9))
 (segment (start 201.795401 151.748382) (end 201.795401 151.777343) (width 1.016) (layer "B.Cu") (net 9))
 (segment (start 203.007133 161.095169) (end 203.007133 160.195074) (width 1.016) (layer "B.Cu") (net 9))
 (segment (start 210.827857 146.409044) (end 206.299422 150.937479) (width 1.016) (layer "B.Cu") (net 9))
 (segment (start 206.299422 150.937479) (end 202.606304 150.937479) (width 1.016) (layer "B.Cu") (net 9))
 (segment (start 203.007133 160.195074) (end 199.639131 156.827072) (width 1.016) (layer "B.Cu") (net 9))
 (segment (start 201.795401 151.777343) (end 196.745672 156.827072) (width 1.016) (layer "B.Cu") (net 9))
 (segment (start 210.827857 129.26287) (end 210.827857 146.409044) (width 1.016) (layer "B.Cu") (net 9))
 (segment (start 203.348436 121.783449) (end 210.827857 129.26287) (width 1.016) (layer "B.Cu") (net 9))
 (segment (start 198.567071 121.783449) (end 203.348436 121.783449) (width 1.016) (layer "B.Cu") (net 9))
 (segment (start 184.807706 139.582967) (end 190.557304 145.332565) (width 1.016) (layer "B.Cu") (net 9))
 (segment (start 199.639131 156.827072) (end 195.482912 156.827072) (width 1.016) (layer "B.Cu") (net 9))
 (segment (start 183.704073 138.494997) (end 184.792043 139.582967) (width 1.016) (layer "B.Cu") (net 9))
 (segment (start 190.557304 145.332565) (end 190.557304 152.304875) (width 1.016) (layer "B.Cu") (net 9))
 (segment (start 183.704073 137.385518) (end 183.704073 138.494997) (width 1.016) (layer "B.Cu") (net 9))
 (segment (start 185.319135 135.770456) (end 183.704073 137.385518) (width 1.016) (layer "B.Cu") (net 9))
 (segment (start 195.482912 156.827072) (end 199.850715 156.827072) (width 1.016) (layer "B.Cu") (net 9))
 (segment (start 202.606304 150.937479) (end 201.795401 151.748382) (width 1.016) (layer "B.Cu") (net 9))
 (segment (start 195.079501 156.827072) (end 195.482912 156.827072) (width 1.016) (layer "B.Cu") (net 9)))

